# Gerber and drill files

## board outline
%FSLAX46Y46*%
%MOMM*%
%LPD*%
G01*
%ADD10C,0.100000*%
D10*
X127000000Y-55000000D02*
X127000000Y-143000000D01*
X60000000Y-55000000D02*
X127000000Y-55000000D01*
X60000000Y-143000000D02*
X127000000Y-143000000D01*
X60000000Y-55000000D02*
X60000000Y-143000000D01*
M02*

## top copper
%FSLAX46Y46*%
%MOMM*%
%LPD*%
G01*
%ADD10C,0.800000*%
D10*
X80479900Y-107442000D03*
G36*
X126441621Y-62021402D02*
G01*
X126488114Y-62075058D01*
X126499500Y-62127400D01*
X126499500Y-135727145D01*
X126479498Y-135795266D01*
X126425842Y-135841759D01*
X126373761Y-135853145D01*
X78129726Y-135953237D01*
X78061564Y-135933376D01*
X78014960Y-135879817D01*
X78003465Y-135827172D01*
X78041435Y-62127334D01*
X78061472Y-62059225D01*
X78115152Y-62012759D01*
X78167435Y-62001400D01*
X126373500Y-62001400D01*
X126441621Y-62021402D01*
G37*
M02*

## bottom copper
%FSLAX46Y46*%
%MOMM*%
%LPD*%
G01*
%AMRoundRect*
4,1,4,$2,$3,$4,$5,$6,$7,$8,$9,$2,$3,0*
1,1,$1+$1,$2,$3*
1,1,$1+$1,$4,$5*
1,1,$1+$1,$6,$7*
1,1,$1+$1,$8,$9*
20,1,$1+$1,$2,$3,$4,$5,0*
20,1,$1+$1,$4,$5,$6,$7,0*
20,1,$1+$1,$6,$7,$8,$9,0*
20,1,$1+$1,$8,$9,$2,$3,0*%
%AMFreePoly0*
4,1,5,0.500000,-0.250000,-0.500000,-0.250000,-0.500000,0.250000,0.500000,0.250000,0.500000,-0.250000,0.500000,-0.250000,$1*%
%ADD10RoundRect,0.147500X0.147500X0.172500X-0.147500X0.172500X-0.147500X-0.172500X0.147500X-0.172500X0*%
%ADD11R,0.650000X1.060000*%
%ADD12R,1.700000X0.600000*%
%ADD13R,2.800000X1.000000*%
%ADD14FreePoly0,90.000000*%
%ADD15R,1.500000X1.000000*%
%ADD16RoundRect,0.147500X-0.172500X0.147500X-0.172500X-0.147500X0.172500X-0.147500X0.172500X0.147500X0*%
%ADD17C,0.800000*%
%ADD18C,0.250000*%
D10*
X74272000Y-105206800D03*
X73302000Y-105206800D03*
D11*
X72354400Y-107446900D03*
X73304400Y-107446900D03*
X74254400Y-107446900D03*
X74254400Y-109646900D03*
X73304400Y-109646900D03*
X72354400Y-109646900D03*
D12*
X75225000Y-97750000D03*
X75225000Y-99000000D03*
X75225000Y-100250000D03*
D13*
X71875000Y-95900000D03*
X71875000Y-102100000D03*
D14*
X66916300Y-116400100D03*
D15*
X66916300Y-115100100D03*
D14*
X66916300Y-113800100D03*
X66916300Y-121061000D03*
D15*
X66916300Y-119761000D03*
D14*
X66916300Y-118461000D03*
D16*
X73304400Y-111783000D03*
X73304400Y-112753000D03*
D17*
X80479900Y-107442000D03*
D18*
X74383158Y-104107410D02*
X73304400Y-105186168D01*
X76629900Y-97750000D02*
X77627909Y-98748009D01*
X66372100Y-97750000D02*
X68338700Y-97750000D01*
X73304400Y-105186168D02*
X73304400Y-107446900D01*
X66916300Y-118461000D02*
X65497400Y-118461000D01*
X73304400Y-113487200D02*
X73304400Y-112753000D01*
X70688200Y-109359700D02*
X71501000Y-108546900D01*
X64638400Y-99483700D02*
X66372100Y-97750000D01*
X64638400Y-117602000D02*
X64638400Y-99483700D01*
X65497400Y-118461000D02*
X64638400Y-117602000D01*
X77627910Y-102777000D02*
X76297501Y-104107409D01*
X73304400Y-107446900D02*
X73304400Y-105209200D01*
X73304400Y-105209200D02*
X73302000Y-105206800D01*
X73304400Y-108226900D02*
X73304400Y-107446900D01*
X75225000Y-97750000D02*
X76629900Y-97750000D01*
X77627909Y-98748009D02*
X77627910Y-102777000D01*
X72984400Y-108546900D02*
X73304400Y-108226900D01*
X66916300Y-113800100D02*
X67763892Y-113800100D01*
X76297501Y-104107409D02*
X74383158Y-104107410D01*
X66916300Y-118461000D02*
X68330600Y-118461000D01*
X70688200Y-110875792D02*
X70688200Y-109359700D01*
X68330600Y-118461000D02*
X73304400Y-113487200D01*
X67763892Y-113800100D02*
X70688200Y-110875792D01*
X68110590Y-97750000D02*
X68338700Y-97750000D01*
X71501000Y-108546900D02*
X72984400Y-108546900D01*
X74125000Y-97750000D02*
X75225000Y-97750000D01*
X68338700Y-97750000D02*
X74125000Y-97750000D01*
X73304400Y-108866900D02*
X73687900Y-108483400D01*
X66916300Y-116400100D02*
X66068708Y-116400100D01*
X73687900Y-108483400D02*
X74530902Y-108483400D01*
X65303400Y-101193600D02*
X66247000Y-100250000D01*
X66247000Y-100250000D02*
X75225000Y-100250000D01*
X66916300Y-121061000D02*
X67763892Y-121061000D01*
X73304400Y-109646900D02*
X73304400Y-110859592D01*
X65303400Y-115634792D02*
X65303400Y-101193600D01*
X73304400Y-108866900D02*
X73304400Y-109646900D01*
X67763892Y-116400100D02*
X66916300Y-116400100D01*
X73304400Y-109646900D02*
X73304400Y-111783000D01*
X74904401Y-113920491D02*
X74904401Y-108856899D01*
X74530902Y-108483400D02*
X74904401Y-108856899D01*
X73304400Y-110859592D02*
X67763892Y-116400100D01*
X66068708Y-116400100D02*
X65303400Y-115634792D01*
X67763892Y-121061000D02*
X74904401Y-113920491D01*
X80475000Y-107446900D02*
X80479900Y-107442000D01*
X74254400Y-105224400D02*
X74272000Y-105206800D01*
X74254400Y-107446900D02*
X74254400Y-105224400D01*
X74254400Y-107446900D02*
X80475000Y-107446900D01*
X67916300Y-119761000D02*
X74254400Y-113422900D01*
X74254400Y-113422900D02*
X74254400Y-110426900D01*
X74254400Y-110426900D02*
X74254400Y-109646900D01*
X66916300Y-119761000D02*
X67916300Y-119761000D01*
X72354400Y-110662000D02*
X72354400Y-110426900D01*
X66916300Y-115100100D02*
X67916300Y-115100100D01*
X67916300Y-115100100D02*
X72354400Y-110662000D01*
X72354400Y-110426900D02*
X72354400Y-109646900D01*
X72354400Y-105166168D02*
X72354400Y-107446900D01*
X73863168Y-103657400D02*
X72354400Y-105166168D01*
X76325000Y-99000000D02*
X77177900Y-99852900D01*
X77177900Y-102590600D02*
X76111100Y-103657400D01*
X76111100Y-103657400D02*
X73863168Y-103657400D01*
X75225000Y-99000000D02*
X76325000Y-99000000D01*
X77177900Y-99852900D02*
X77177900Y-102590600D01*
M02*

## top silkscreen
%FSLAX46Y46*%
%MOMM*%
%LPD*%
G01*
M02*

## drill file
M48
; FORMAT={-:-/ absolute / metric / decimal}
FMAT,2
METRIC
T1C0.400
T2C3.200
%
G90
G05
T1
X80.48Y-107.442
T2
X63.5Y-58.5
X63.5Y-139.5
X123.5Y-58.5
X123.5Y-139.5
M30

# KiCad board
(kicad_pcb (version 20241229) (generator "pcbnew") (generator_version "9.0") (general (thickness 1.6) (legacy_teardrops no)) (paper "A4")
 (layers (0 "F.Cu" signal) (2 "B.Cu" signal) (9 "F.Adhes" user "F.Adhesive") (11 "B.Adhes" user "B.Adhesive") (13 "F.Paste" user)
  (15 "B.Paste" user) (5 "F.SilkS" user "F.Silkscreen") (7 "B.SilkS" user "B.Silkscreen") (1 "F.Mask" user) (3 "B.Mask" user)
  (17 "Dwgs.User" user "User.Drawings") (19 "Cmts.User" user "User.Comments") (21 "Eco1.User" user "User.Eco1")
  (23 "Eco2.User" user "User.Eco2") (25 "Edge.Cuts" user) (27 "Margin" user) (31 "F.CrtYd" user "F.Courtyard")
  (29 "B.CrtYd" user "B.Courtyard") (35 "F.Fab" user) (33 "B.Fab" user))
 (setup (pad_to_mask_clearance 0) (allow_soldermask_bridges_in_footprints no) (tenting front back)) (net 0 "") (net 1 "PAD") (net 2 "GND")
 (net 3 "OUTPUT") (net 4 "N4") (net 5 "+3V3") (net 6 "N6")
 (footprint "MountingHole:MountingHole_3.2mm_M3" (layer "F.Cu") (at 63.5 58.5)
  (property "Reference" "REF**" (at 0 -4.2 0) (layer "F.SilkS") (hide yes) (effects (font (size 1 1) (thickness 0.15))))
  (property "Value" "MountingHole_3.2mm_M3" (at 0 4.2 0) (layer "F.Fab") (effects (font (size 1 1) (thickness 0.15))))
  (pad "" np_thru_hole circle (at 0 0) (size 3.2 3.2) (drill 3.2) (layers "*.Cu" "*.Mask")))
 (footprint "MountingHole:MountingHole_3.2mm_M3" (layer "F.Cu") (at 63.5 139.5)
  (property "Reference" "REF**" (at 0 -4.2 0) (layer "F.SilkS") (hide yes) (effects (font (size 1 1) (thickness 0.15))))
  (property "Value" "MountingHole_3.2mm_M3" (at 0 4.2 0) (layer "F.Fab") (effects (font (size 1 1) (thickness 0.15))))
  (pad "" np_thru_hole circle (at 0 0) (size 3.2 3.2) (drill 3.2) (layers "*.Cu" "*.Mask")))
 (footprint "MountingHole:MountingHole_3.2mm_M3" (layer "F.Cu") (at 123.5 58.5)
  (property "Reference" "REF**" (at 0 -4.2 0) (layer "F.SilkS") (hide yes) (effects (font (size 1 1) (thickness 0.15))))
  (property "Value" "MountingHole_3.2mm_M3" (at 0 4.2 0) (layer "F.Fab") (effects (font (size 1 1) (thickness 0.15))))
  (pad "" np_thru_hole circle (at 0 0) (size 3.2 3.2) (drill 3.2) (layers "*.Cu" "*.Mask")))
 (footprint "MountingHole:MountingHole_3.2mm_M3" (layer "F.Cu") (at 123.5 139.5)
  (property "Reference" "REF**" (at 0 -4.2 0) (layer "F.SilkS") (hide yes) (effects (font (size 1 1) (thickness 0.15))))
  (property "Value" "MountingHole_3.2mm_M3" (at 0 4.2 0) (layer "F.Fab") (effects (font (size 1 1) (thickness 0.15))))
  (pad "" np_thru_hole circle (at 0 0) (size 3.2 3.2) (drill 3.2) (layers "*.Cu" "*.Mask")))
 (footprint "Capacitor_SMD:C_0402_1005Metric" (layer "B.Cu") (at 73.787 105.2068 180)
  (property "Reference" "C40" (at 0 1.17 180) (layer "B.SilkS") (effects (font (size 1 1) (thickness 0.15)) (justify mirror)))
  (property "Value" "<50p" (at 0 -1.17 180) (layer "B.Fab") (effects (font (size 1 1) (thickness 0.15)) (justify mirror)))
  (pad "1" smd roundrect (at -0.485 0 180) (size 0.59 0.64) (layers "B.Cu" "B.Mask" "B.Paste") (roundrect_rratio 0.25) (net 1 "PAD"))
  (pad "2" smd roundrect (at 0.485 0 180) (size 0.59 0.64) (layers "B.Cu" "B.Mask" "B.Paste") (roundrect_rratio 0.25) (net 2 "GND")))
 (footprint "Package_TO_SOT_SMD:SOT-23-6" (layer "B.Cu") (at 73.3044 108.5469 -90)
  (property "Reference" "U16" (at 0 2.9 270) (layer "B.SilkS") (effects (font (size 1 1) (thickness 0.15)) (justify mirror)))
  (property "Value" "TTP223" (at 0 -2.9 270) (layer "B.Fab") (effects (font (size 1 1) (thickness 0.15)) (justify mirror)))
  (pad "1" smd rect (at -1.1 0.95 270) (size 1.06 0.65) (layers "B.Cu" "B.Mask" "B.Paste") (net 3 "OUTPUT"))
  (pad "2" smd rect (at -1.1 0 270) (size 1.06 0.65) (layers "B.Cu" "B.Mask" "B.Paste") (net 2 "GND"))
  (pad "3" smd rect (at -1.1 -0.95 270) (size 1.06 0.65) (layers "B.Cu" "B.Mask" "B.Paste") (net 1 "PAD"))
  (pad "4" smd rect (at 1.1 -0.95 270) (size 1.06 0.65) (layers "B.Cu" "B.Mask" "B.Paste") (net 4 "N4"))
  (pad "5" smd rect (at 1.1 0 270) (size 1.06 0.65) (layers "B.Cu" "B.Mask" "B.Paste") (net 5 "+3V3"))
  (pad "6" smd rect (at 1.1 0.95 270) (size 1.06 0.65) (layers "B.Cu" "B.Mask" "B.Paste") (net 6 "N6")))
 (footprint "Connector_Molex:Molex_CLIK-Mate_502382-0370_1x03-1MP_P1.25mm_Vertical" (layer "B.Cu") (at 73.275 99 -90)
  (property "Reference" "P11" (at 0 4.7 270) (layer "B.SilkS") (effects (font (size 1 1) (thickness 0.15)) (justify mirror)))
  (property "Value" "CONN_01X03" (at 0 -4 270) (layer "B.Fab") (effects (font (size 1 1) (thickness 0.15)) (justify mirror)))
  (pad "1" smd rect (at -1.25 -1.95 270) (size 0.6 1.7) (layers "B.Cu" "B.Mask" "B.Paste") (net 2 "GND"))
  (pad "2" smd rect (at 0 -1.95 270) (size 0.6 1.7) (layers "B.Cu" "B.Mask" "B.Paste") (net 3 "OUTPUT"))
  (pad "3" smd rect (at 1.25 -1.95 270) (size 0.6 1.7) (layers "B.Cu" "B.Mask" "B.Paste") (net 5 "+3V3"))
  (pad "MP" smd rect (at -3.1 1.4 270) (size 1 2.8) (layers "B.Cu" "B.Mask" "B.Paste"))
  (pad "MP" smd rect (at 3.1 1.4 270) (size 1 2.8) (layers "B.Cu" "B.Mask" "B.Paste")))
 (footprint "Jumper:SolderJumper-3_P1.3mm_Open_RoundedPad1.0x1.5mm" (layer "B.Cu") (at 66.9163 115.1001 90)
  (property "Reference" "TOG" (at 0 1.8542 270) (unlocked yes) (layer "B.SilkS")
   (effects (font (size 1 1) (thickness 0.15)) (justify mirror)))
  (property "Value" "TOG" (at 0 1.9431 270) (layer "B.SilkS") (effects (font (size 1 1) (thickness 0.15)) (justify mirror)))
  (pad "1" smd custom (at -1.3 0 90) (size 1 0.5) (layers "B.Cu" "B.Mask") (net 5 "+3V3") (zone_connect 0)
   (options (clearance outline) (anchor rect)) (primitives))
  (pad "2" smd rect (at 0 0 90) (size 1 1.5) (layers "B.Cu" "B.Mask") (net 6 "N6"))
  (pad "3" smd custom (at 1.3 0 90) (size 1 0.5) (layers "B.Cu" "B.Mask") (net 2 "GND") (zone_connect 0)
   (options (clearance outline) (anchor rect)) (primitives)))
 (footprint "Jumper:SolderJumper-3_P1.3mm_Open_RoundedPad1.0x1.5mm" (layer "B.Cu") (at 66.9163 119.761 90)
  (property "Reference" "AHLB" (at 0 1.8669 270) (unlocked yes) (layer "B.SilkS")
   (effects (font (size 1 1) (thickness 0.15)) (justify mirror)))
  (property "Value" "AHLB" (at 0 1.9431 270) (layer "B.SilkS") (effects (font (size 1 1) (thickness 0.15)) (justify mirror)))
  (pad "1" smd custom (at -1.3 0 90) (size 1 0.5) (layers "B.Cu" "B.Mask") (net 5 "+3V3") (zone_connect 0)
   (options (clearance outline) (anchor rect)) (primitives))
  (pad "2" smd rect (at 0 0 90) (size 1 1.5) (layers "B.Cu" "B.Mask") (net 4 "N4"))
  (pad "3" smd custom (at 1.3 0 90) (size 1 0.5) (layers "B.Cu" "B.Mask") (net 2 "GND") (zone_connect 0)
   (options (clearance outline) (anchor rect)) (primitives)))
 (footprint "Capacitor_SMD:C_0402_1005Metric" (layer "B.Cu") (at 73.3044 112.268 -90)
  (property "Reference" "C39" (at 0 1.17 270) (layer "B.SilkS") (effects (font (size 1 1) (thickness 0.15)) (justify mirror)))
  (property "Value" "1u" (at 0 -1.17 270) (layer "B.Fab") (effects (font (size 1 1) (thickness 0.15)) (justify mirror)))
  (pad "1" smd roundrect (at -0.485 0 270) (size 0.59 0.64) (layers "B.Cu" "B.Mask" "B.Paste") (roundrect_rratio 0.25) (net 5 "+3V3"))
  (pad "2" smd roundrect (at 0.485 0 270) (size 0.59 0.64) (layers "B.Cu" "B.Mask" "B.Paste") (roundrect_rratio 0.25) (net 2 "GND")))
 (gr_line (start 127 55) (end 127 143) (stroke (width 0.1) (type solid)) (layer "Edge.Cuts"))
 (gr_line (start 60 55) (end 127 55) (stroke (width 0.1) (type solid)) (layer "Edge.Cuts"))
 (gr_line (start 60 143) (end 127 143) (stroke (width 0.1) (type solid)) (layer "Edge.Cuts"))
 (gr_line (start 60 55) (end 60 143) (stroke (width 0.1) (type solid)) (layer "Edge.Cuts"))
 (segment (start 74.383158 104.10741) (end 73.3044 105.186168) (width 0.25) (layer "B.Cu") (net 2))
 (segment (start 76.6299 97.75) (end 77.627909 98.748009) (width 0.25) (layer "B.Cu") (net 2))
 (segment (start 66.3721 97.75) (end 68.3387 97.75) (width 0.25) (layer "B.Cu") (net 2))
 (segment (start 73.3044 105.186168) (end 73.3044 107.4469) (width 0.25) (layer "B.Cu") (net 2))
 (segment (start 66.9163 118.461) (end 65.4974 118.461) (width 0.25) (layer "B.Cu") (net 2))
 (segment (start 73.3044 113.4872) (end 73.3044 112.753) (width 0.25) (layer "B.Cu") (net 2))
 (segment (start 70.6882 109.3597) (end 71.501 108.5469) (width 0.25) (layer "B.Cu") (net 2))
 (segment (start 64.6384 99.4837) (end 66.3721 97.75) (width 0.25) (layer "B.Cu") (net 2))
 (segment (start 64.6384 117.602) (end 64.6384 99.4837) (width 0.25) (layer "B.Cu") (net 2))
 (segment (start 65.4974 118.461) (end 64.6384 117.602) (width 0.25) (layer "B.Cu") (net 2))
 (segment (start 77.62791 102.777) (end 76.297501 104.107409) (width 0.25) (layer "B.Cu") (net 2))
 (segment (start 73.3044 107.4469) (end 73.3044 105.2092) (width 0.25) (layer "B.Cu") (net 2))
 (segment (start 73.3044 105.2092) (end 73.302 105.2068) (width 0.25) (layer "B.Cu") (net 2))
 (segment (start 73.3044 108.2269) (end 73.3044 107.4469) (width 0.25) (layer "B.Cu") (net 2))
 (segment (start 75.225 97.75) (end 76.6299 97.75) (width 0.25) (layer "B.Cu") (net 2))
 (segment (start 77.627909 98.748009) (end 77.62791 102.777) (width 0.25) (layer "B.Cu") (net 2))
 (segment (start 72.9844 108.5469) (end 73.3044 108.2269) (width 0.25) (layer "B.Cu") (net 2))
 (segment (start 66.9163 113.8001) (end 67.763892 113.8001) (width 0.25) (layer "B.Cu") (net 2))
 (segment (start 76.297501 104.107409) (end 74.383158 104.10741) (width 0.25) (layer "B.Cu") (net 2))
 (segment (start 66.9163 118.461) (end 68.3306 118.461) (width 0.25) (layer "B.Cu") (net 2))
 (segment (start 70.6882 110.875792) (end 70.6882 109.3597) (width 0.25) (layer "B.Cu") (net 2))
 (segment (start 68.3306 118.461) (end 73.3044 113.4872) (width 0.25) (layer "B.Cu") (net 2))
 (segment (start 67.763892 113.8001) (end 70.6882 110.875792) (width 0.25) (layer "B.Cu") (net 2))
 (segment (start 68.11059 97.75) (end 68.3387 97.75) (width 0.25) (layer "B.Cu") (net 2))
 (segment (start 71.501 108.5469) (end 72.9844 108.5469) (width 0.25) (layer "B.Cu") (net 2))
 (segment (start 74.125 97.75) (end 75.225 97.75) (width 0.25) (layer "B.Cu") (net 2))
 (segment (start 68.3387 97.75) (end 74.125 97.75) (width 0.25) (layer "B.Cu") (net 2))
 (segment (start 73.3044 108.8669) (end 73.6879 108.4834) (width 0.25) (layer "B.Cu") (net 5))
 (segment (start 66.9163 116.4001) (end 66.068708 116.4001) (width 0.25) (layer "B.Cu") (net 5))
 (segment (start 73.6879 108.4834) (end 74.530902 108.4834) (width 0.25) (layer "B.Cu") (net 5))
 (segment (start 65.3034 101.1936) (end 66.247 100.25) (width 0.25) (layer "B.Cu") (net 5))
 (segment (start 66.247 100.25) (end 75.225 100.25) (width 0.25) (layer "B.Cu") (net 5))
 (segment (start 66.9163 121.061) (end 67.763892 121.061) (width 0.25) (layer "B.Cu") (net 5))
 (segment (start 73.3044 109.6469) (end 73.3044 110.859592) (width 0.25) (layer "B.Cu") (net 5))
 (segment (start 65.3034 115.634792) (end 65.3034 101.1936) (width 0.25) (layer "B.Cu") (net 5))
 (segment (start 73.3044 108.8669) (end 73.3044 109.6469) (width 0.25) (layer "B.Cu") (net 5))
 (segment (start 67.763892 116.4001) (end 66.9163 116.4001) (width 0.25) (layer "B.Cu") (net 5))
 (segment (start 73.3044 109.6469) (end 73.3044 111.783) (width 0.25) (layer "B.Cu") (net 5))
 (segment (start 74.904401 113.920491) (end 74.904401 108.856899) (width 0.25) (layer "B.Cu") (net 5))
 (segment (start 74.530902 108.4834) (end 74.904401 108.856899) (width 0.25) (layer "B.Cu") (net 5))
 (segment (start 73.3044 110.859592) (end 67.763892 116.4001) (width 0.25) (layer "B.Cu") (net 5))
 (segment (start 66.068708 116.4001) (end 65.3034 115.634792) (width 0.25) (layer "B.Cu") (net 5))
 (segment (start 67.763892 121.061) (end 74.904401 113.920491) (width 0.25) (layer "B.Cu") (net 5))
 (via (at 80.4799 107.442) (size 0.8) (drill 0.4) (layers "F.Cu" "B.Cu") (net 1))
 (segment (start 80.475 107.4469) (end 80.4799 107.442) (width 0.25) (layer "B.Cu") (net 1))
 (segment (start 74.2544 105.2244) (end 74.272 105.2068) (width 0.25) (layer "B.Cu") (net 1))
 (segment (start 74.2544 107.4469) (end 74.2544 105.2244) (width 0.25) (layer "B.Cu") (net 1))
 (segment (start 74.2544 107.4469) (end 80.475 107.4469) (width 0.25) (layer "B.Cu") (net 1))
 (segment (start 67.9163 119.761) (end 74.2544 113.4229) (width 0.25) (layer "B.Cu") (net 4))
 (segment (start 74.2544 113.4229) (end 74.2544 110.4269) (width 0.25) (layer "B.Cu") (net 4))
 (segment (start 74.2544 110.4269) (end 74.2544 109.6469) (width 0.25) (layer "B.Cu") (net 4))
 (segment (start 66.9163 119.761) (end 67.9163 119.761) (width 0.25) (layer "B.Cu") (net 4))
 (segment (start 72.3544 110.662) (end 72.3544 110.4269) (width 0.25) (layer "B.Cu") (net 6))
 (segment (start 66.9163 115.1001) (end 67.9163 115.1001) (width 0.25) (layer "B.Cu") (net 6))
 (segment (start 67.9163 115.1001) (end 72.3544 110.662) (width 0.25) (layer "B.Cu") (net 6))
 (segment (start 72.3544 110.4269) (end 72.3544 109.6469) (width 0.25) (layer "B.Cu") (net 6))
 (segment (start 72.3544 105.166168) (end 72.3544 107.4469) (width 0.25) (layer "B.Cu") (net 3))
 (segment (start 73.863168 103.6574) (end 72.3544 105.166168) (width 0.25) (layer "B.Cu") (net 3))
 (segment (start 76.325 99) (end 77.1779 99.8529) (width 0.25) (layer "B.Cu") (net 3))
 (segment (start 77.1779 102.5906) (end 76.1111 103.6574) (width 0.25) (layer "B.Cu") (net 3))
 (segment (start 76.1111 103.6574) (end 73.863168 103.6574) (width 0.25) (layer "B.Cu") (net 3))
 (segment (start 75.225 99) (end 76.325 99) (width 0.25) (layer "B.Cu") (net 3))
 (segment (start 77.1779 99.8529) (end 77.1779 102.5906) (width 0.25) (layer "B.Cu") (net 3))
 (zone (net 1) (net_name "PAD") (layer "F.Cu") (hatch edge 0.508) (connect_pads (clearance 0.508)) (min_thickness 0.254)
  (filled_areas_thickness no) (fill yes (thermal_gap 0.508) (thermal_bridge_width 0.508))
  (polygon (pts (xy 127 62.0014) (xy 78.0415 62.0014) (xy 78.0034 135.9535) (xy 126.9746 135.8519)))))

